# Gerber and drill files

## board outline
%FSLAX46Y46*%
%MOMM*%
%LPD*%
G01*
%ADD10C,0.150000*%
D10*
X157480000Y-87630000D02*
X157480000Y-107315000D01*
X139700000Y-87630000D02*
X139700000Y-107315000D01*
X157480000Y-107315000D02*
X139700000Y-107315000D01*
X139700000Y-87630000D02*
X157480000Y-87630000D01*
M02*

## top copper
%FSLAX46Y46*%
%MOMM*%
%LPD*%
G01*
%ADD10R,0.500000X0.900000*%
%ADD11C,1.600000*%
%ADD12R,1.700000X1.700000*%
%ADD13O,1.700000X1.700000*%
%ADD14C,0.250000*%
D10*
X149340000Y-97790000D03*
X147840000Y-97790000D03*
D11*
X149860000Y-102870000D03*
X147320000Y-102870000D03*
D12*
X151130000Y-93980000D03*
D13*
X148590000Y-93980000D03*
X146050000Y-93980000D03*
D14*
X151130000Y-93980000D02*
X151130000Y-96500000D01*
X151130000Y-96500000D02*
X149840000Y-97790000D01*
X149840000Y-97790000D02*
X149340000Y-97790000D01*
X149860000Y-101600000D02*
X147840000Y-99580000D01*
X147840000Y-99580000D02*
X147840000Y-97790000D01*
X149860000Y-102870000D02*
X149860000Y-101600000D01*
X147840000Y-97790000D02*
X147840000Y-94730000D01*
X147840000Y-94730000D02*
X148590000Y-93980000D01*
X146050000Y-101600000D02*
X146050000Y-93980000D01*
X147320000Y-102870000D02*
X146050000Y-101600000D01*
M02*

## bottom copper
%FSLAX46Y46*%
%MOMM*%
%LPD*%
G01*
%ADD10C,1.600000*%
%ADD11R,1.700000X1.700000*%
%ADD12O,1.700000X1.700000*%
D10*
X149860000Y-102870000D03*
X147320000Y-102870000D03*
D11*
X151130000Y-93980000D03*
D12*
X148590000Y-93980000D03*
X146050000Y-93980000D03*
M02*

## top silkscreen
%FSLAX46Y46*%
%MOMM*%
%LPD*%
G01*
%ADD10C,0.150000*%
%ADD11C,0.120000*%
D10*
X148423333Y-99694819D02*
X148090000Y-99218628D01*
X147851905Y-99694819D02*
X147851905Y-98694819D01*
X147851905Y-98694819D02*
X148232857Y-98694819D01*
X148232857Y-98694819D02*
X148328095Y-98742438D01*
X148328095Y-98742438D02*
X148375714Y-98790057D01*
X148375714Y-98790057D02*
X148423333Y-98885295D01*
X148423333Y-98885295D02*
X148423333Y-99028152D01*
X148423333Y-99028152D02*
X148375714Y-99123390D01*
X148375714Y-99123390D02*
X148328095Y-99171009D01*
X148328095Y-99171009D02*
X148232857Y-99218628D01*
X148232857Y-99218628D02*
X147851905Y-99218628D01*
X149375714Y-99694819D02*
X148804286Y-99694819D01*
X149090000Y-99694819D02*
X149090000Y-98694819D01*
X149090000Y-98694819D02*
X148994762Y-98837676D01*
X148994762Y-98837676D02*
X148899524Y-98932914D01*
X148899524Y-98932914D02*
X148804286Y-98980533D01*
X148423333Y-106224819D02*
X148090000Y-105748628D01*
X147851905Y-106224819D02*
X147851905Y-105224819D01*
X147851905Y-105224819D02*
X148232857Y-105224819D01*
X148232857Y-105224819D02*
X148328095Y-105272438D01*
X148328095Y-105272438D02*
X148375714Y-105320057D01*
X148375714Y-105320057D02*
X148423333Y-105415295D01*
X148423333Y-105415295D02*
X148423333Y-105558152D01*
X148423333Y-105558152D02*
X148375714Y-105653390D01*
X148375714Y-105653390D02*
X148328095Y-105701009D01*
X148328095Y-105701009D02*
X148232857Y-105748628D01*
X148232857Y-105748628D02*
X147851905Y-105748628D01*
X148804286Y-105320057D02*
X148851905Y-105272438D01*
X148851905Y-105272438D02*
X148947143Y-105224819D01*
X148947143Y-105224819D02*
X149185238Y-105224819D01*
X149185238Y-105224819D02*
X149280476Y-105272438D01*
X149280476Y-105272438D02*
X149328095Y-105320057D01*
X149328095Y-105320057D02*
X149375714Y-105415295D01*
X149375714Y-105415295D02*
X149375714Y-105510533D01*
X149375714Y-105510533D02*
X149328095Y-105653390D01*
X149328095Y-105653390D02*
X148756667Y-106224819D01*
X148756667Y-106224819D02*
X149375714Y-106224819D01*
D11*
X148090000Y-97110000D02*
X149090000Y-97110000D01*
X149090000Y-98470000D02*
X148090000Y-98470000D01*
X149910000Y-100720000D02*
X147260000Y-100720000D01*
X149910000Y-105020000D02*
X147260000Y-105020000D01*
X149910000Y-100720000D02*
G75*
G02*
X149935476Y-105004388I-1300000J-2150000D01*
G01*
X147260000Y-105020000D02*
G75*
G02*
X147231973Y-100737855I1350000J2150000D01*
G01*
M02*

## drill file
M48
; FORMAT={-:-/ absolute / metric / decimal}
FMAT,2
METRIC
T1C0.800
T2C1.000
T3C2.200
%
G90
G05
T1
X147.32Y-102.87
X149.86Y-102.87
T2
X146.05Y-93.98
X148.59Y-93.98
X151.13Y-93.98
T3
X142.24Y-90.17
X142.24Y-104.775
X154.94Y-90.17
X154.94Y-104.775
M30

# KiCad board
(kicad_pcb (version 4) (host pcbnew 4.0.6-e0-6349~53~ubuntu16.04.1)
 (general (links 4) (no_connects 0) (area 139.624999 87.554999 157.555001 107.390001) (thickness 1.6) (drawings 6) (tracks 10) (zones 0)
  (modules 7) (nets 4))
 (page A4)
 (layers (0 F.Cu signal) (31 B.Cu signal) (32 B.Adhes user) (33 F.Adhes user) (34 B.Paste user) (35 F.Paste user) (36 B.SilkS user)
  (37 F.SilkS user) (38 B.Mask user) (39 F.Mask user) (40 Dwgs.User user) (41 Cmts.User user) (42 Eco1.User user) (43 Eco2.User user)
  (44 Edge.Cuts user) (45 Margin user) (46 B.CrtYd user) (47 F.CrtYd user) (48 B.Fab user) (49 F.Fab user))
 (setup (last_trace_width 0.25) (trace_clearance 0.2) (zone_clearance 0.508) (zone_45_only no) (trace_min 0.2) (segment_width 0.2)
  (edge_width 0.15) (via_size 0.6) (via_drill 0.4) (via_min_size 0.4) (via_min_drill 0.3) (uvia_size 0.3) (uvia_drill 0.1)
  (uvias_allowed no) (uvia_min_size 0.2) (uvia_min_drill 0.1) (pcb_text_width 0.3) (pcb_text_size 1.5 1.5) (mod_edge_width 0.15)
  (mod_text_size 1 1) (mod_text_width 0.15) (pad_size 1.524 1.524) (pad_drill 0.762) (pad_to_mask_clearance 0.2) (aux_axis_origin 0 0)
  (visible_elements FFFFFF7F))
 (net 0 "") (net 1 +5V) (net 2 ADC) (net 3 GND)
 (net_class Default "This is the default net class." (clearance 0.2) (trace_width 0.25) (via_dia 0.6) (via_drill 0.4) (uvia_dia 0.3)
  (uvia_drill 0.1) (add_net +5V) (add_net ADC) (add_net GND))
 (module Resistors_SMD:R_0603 (layer F.Cu) (at 148.59 97.79 180)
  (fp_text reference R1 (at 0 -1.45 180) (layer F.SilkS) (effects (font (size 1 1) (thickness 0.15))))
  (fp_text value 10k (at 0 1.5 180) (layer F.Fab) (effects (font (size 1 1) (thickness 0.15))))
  (fp_line (start 0.5 0.68) (end -0.5 0.68) (layer F.SilkS) (width 0.12))
  (fp_line (start -0.5 -0.68) (end 0.5 -0.68) (layer F.SilkS) (width 0.12))
  (pad 1 smd rect (at -0.75 0 180) (size 0.5 0.9) (layers F.Cu F.Paste F.Mask) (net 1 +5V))
  (pad 2 smd rect (at 0.75 0 180) (size 0.5 0.9) (layers F.Cu F.Paste F.Mask) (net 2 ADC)))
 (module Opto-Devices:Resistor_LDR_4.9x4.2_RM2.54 (layer F.Cu) (at 149.86 102.87 180)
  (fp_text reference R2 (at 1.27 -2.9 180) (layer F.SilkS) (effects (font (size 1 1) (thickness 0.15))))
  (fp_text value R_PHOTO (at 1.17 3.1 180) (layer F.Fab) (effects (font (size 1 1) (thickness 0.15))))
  (fp_line (start -0.05 2.15) (end 2.6 2.15) (layer F.SilkS) (width 0.12))
  (fp_line (start -0.05 -2.15) (end 2.6 -2.15) (layer F.SilkS) (width 0.12))
  (fp_arc (start 1.25 0) (end -0.05 2.15) (angle 117) (layer F.SilkS) (width 0.12))
  (fp_arc (start 1.25 0) (end 2.6 -2.15) (angle 115) (layer F.SilkS) (width 0.12))
  (pad 1 thru_hole circle (at 0 0 180) (size 1.6 1.6) (drill 0.8) (layers *.Cu *.Mask) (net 2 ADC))
  (pad 2 thru_hole circle (at 2.54 0 180) (size 1.6 1.6) (drill 0.8) (layers *.Cu *.Mask) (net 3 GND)))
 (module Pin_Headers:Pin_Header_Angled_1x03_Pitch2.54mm (layer B.Cu) (at 151.13 93.98 90)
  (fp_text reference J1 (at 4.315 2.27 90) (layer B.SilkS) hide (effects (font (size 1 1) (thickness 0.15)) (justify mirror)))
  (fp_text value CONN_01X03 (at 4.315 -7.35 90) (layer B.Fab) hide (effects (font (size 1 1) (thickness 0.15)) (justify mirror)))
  (pad 1 thru_hole rect (at 0 0 90) (size 1.7 1.7) (drill 1) (layers *.Cu *.Mask) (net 1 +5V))
  (pad 2 thru_hole oval (at 0 -2.54 90) (size 1.7 1.7) (drill 1) (layers *.Cu *.Mask) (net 2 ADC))
  (pad 3 thru_hole oval (at 0 -5.08 90) (size 1.7 1.7) (drill 1) (layers *.Cu *.Mask) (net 3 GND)))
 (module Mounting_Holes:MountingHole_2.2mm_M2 (layer F.Cu) (at 154.94 90.17)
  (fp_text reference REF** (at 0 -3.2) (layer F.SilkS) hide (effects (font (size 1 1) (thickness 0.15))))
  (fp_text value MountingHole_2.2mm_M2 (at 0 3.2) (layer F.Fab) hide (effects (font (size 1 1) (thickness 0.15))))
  (pad 1 np_thru_hole circle (at 0 0) (size 2.2 2.2) (drill 2.2) (layers *.Cu *.Mask)))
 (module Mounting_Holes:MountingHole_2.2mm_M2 (layer F.Cu) (at 142.24 90.17)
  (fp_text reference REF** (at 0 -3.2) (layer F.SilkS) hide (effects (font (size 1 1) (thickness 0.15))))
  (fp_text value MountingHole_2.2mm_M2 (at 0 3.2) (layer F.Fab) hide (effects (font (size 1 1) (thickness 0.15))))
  (pad 1 np_thru_hole circle (at 0 0) (size 2.2 2.2) (drill 2.2) (layers *.Cu *.Mask)))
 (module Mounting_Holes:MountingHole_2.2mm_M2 (layer F.Cu) (at 142.24 104.775)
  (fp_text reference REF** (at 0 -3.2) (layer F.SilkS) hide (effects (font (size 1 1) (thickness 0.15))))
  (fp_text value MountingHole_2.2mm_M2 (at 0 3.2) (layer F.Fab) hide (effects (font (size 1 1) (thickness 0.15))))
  (pad 1 np_thru_hole circle (at 0 0) (size 2.2 2.2) (drill 2.2) (layers *.Cu *.Mask)))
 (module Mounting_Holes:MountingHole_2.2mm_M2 (layer F.Cu) (at 154.94 104.775)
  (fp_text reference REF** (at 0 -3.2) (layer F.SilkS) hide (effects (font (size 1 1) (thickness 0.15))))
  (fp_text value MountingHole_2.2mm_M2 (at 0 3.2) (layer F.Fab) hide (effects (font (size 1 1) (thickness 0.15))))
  (pad 1 np_thru_hole circle (at 0 0) (size 2.2 2.2) (drill 2.2) (layers *.Cu *.Mask)))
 (gr_line (start 157.48 87.63) (end 157.48 107.315) (layer Edge.Cuts) (width 0.15))
 (gr_line (start 139.7 87.63) (end 139.7 107.315) (layer Edge.Cuts) (width 0.15))
 (gr_line (start 157.48 107.315) (end 139.7 107.315) (layer Edge.Cuts) (width 0.15))
 (gr_line (start 139.7 87.63) (end 157.48 87.63) (layer Edge.Cuts) (width 0.15))
 (segment (start 151.13 93.98) (end 151.13 96.5) (width 0.25) (layer F.Cu) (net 1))
 (segment (start 151.13 96.5) (end 149.84 97.79) (width 0.25) (layer F.Cu) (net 1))
 (segment (start 149.84 97.79) (end 149.34 97.79) (width 0.25) (layer F.Cu) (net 1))
 (segment (start 149.86 101.6) (end 147.84 99.58) (width 0.25) (layer F.Cu) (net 2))
 (segment (start 147.84 99.58) (end 147.84 97.79) (width 0.25) (layer F.Cu) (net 2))
 (segment (start 149.86 102.87) (end 149.86 101.6) (width 0.25) (layer F.Cu) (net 2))
 (segment (start 147.84 97.79) (end 147.84 94.73) (width 0.25) (layer F.Cu) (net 2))
 (segment (start 147.84 94.73) (end 148.59 93.98) (width 0.25) (layer F.Cu) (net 2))
 (segment (start 146.05 101.6) (end 146.05 93.98) (width 0.25) (layer F.Cu) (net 3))
 (segment (start 147.32 102.87) (end 146.05 101.6) (width 0.25) (layer F.Cu) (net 3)))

